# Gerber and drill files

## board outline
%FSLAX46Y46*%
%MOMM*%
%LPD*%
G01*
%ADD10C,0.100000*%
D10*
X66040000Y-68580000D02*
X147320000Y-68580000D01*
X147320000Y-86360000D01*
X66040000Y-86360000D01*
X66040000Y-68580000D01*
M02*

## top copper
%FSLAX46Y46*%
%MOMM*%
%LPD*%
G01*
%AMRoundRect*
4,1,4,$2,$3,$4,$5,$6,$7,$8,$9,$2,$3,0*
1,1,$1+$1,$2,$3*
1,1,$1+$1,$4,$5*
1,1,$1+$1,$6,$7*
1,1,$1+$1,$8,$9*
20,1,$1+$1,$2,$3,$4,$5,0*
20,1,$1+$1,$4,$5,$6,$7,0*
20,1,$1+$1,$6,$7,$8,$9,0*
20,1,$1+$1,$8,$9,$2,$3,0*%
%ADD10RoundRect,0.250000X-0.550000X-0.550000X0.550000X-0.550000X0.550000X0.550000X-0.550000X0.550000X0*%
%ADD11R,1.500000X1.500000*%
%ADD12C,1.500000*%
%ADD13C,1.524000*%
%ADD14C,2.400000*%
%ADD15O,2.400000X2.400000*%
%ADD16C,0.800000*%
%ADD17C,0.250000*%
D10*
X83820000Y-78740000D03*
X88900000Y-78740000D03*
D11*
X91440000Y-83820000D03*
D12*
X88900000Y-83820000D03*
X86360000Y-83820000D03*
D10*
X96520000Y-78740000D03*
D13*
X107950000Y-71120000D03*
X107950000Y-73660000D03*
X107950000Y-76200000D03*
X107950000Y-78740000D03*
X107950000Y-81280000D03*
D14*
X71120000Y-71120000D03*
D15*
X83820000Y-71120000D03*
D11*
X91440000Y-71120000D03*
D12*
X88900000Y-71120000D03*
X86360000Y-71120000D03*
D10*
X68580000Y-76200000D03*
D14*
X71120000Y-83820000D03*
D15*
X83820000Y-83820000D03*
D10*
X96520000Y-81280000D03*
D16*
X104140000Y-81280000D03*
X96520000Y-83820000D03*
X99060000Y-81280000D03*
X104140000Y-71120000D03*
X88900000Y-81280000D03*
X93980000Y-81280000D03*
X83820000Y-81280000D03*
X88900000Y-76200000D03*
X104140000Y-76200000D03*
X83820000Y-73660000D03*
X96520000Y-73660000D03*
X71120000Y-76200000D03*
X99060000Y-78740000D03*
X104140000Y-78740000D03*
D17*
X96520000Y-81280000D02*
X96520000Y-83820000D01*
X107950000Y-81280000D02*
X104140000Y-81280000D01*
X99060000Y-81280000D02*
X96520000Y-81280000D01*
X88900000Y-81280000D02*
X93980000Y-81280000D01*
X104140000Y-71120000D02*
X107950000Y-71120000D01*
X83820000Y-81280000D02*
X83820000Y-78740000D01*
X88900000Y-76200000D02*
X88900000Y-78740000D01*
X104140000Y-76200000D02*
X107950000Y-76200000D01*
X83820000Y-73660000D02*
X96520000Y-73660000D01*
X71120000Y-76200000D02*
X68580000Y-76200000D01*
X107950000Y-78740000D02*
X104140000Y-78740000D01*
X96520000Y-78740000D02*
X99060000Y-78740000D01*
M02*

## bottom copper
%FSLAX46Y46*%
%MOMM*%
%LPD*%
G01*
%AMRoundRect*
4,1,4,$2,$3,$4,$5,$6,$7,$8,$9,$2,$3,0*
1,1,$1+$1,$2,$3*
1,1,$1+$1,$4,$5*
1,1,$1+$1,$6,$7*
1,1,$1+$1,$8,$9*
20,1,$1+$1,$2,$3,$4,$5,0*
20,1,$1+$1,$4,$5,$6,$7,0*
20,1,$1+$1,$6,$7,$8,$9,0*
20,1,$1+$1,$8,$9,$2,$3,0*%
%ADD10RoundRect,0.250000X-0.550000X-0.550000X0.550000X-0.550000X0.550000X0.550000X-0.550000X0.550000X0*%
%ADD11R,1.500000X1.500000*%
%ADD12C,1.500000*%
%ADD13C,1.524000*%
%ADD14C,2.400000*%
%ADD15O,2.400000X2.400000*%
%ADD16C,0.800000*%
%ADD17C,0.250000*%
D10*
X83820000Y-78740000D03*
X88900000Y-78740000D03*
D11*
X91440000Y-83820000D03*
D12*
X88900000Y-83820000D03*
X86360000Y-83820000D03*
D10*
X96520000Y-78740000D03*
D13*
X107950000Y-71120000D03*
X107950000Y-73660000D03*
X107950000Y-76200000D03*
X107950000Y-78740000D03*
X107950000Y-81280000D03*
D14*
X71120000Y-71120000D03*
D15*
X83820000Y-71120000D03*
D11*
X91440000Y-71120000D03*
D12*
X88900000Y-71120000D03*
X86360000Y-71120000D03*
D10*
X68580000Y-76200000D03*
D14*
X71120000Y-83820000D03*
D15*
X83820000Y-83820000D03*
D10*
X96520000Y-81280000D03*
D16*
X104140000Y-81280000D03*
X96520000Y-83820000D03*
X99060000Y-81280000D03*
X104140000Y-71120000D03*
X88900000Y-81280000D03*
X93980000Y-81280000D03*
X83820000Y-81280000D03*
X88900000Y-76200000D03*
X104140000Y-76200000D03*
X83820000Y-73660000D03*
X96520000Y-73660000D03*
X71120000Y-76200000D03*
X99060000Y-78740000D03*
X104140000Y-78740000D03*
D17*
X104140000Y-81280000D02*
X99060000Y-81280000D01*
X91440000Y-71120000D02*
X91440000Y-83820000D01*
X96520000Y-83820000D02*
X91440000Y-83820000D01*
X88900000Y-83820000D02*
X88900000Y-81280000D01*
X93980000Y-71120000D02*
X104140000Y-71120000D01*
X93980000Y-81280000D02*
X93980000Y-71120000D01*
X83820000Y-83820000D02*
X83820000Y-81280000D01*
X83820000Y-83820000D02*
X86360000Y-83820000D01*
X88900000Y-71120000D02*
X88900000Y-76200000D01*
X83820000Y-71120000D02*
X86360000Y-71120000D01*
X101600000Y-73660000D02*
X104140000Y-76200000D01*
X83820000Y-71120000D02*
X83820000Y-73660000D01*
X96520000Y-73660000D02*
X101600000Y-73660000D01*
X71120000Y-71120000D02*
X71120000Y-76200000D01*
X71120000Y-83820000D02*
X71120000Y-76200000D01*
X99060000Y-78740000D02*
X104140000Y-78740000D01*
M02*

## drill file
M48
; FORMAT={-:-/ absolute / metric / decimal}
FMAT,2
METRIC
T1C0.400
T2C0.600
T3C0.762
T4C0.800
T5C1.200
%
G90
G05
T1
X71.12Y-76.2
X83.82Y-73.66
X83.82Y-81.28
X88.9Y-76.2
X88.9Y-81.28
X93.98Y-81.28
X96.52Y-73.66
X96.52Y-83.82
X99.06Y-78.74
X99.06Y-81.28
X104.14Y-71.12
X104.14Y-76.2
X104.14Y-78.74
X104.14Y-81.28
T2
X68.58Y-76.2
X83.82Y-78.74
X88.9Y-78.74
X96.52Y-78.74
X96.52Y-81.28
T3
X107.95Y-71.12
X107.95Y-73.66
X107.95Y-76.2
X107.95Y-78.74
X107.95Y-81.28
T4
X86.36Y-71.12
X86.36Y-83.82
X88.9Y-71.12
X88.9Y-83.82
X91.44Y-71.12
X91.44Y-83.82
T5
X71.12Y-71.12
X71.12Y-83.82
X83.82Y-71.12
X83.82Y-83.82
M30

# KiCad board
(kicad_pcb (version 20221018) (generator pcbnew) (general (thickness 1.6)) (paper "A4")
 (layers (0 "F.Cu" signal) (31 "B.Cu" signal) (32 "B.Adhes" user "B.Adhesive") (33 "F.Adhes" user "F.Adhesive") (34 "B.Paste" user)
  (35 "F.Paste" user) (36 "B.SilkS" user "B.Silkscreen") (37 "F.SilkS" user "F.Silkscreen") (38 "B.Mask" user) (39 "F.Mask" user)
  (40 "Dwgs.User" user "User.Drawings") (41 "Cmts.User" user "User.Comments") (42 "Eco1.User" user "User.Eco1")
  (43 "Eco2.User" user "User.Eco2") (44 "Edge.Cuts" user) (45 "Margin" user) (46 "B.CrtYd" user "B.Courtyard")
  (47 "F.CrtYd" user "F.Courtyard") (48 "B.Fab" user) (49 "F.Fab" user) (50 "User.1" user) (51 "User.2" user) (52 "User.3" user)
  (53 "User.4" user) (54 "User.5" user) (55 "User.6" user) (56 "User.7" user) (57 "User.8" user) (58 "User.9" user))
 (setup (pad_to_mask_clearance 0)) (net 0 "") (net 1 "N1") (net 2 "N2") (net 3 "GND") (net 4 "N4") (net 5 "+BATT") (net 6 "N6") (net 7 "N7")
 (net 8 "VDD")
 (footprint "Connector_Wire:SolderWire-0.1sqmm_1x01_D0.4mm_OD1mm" (layer "F.Cu") (at 83.82 78.74)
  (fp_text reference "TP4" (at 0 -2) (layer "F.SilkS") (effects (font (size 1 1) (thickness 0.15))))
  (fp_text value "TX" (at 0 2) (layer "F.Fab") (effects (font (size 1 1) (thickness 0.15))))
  (pad "1" thru_hole roundrect (at 0 0) (size 1.6 1.6) (drill 0.6) (layers "*.Cu" "*.Mask") (roundrect_rratio 0.15625) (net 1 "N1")))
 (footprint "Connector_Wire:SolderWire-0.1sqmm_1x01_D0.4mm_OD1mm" (layer "F.Cu") (at 88.9 78.74)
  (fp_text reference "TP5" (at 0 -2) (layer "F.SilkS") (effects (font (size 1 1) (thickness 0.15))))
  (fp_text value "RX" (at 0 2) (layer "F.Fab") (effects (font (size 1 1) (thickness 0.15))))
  (pad "1" thru_hole roundrect (at 0 0) (size 1.6 1.6) (drill 0.6) (layers "*.Cu" "*.Mask") (roundrect_rratio 0.15625) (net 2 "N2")))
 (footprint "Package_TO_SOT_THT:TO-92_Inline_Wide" (layer "F.Cu") (at 91.44 83.82 180)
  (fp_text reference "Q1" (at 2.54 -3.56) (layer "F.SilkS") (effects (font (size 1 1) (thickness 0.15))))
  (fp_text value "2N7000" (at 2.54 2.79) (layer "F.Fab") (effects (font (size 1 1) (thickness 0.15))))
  (pad "1" thru_hole rect (at 0 0 180) (size 1.5 1.5) (drill 0.8) (layers "*.Cu" "*.Mask") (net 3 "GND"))
  (pad "2" thru_hole circle (at 2.54 0 180) (size 1.5 1.5) (drill 0.8) (layers "*.Cu" "*.Mask") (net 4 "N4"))
  (pad "3" thru_hole circle (at 5.08 0 180) (size 1.5 1.5) (drill 0.8) (layers "*.Cu" "*.Mask") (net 1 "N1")))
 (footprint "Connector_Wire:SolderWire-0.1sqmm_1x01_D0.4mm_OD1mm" (layer "F.Cu") (at 96.52 78.74)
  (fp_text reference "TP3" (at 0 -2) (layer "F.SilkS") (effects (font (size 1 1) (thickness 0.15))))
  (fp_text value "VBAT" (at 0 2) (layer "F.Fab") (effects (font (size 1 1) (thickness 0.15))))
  (pad "1" thru_hole roundrect (at 0 0) (size 1.6 1.6) (drill 0.6) (layers "*.Cu" "*.Mask") (roundrect_rratio 0.15625) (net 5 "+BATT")))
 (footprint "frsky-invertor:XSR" (layer "F.Cu") (at 107.95 71.12)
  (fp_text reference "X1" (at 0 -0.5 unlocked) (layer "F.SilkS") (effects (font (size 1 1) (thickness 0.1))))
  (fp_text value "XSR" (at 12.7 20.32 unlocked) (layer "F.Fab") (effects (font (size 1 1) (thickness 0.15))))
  (pad "1" thru_hole circle (at 0 0) (size 1.524 1.524) (drill 0.762) (layers "*.Cu" "*.Mask") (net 4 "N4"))
  (pad "2" thru_hole circle (at 0 2.54) (size 1.524 1.524) (drill 0.762) (layers "*.Cu" "*.Mask") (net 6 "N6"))
  (pad "3" thru_hole circle (at 0 5.08) (size 1.524 1.524) (drill 0.762) (layers "*.Cu" "*.Mask") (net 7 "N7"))
  (pad "4" thru_hole circle (at 0 7.62) (size 1.524 1.524) (drill 0.762) (layers "*.Cu" "*.Mask") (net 5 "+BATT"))
  (pad "5" thru_hole circle (at 0 10.16) (size 1.524 1.524) (drill 0.762) (layers "*.Cu" "*.Mask") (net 3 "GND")))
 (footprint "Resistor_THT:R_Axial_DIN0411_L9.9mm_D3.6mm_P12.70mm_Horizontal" (layer "F.Cu") (at 71.12 71.12)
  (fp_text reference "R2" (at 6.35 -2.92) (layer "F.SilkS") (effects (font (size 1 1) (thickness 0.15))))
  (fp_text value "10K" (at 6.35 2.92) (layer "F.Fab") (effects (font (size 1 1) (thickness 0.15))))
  (pad "1" thru_hole circle (at 0 0) (size 2.4 2.4) (drill 1.2) (layers "*.Cu" "*.Mask") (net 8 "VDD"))
  (pad "2" thru_hole oval (at 12.7 0) (size 2.4 2.4) (drill 1.2) (layers "*.Cu" "*.Mask") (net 7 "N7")))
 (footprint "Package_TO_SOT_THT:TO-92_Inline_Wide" (layer "F.Cu") (at 91.44 71.12 180)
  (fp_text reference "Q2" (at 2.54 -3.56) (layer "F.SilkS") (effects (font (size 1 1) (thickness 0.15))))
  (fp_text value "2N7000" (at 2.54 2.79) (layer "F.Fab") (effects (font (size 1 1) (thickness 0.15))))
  (pad "1" thru_hole rect (at 0 0 180) (size 1.5 1.5) (drill 0.8) (layers "*.Cu" "*.Mask") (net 3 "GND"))
  (pad "2" thru_hole circle (at 2.54 0 180) (size 1.5 1.5) (drill 0.8) (layers "*.Cu" "*.Mask") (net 2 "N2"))
  (pad "3" thru_hole circle (at 5.08 0 180) (size 1.5 1.5) (drill 0.8) (layers "*.Cu" "*.Mask") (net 7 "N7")))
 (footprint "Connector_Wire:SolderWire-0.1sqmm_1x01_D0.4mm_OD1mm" (layer "F.Cu") (at 68.58 76.2)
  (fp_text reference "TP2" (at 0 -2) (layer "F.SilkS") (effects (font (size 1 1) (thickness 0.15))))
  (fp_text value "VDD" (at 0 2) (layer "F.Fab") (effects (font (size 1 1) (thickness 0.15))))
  (pad "1" thru_hole roundrect (at 0 0) (size 1.6 1.6) (drill 0.6) (layers "*.Cu" "*.Mask") (roundrect_rratio 0.15625) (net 8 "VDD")))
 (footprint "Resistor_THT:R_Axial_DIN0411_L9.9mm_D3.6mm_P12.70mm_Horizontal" (layer "F.Cu") (at 71.12 83.82)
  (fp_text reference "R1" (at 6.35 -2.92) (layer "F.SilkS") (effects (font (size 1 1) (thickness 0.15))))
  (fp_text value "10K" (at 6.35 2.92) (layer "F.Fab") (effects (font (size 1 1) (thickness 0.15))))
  (pad "1" thru_hole circle (at 0 0) (size 2.4 2.4) (drill 1.2) (layers "*.Cu" "*.Mask") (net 8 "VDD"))
  (pad "2" thru_hole oval (at 12.7 0) (size 2.4 2.4) (drill 1.2) (layers "*.Cu" "*.Mask") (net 1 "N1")))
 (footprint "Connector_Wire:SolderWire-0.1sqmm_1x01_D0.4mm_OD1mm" (layer "F.Cu") (at 96.52 81.28)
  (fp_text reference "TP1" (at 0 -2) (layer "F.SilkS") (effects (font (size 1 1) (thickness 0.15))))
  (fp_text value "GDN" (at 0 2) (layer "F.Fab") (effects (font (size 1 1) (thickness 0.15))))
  (pad "1" thru_hole roundrect (at 0 0) (size 1.6 1.6) (drill 0.6) (layers "*.Cu" "*.Mask") (roundrect_rratio 0.15625) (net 3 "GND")))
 (gr_rect (start 66.04 68.58) (end 147.32 86.36) (stroke (width 0.1) (type default)) (fill none) (layer "Edge.Cuts"))
 (segment (start 96.52 81.28) (end 96.52 83.82) (width 0.25) (layer "F.Cu") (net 3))
 (segment (start 107.95 81.28) (end 104.14 81.28) (width 0.25) (layer "F.Cu") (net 3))
 (segment (start 99.06 81.28) (end 96.52 81.28) (width 0.25) (layer "F.Cu") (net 3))
 (via (at 104.14 81.28) (size 0.8) (drill 0.4) (layers "F.Cu" "B.Cu") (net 3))
 (via (at 96.52 83.82) (size 0.8) (drill 0.4) (layers "F.Cu" "B.Cu") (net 3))
 (via (at 99.06 81.28) (size 0.8) (drill 0.4) (layers "F.Cu" "B.Cu") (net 3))
 (segment (start 104.14 81.28) (end 99.06 81.28) (width 0.25) (layer "B.Cu") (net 3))
 (segment (start 91.44 71.12) (end 91.44 83.82) (width 0.25) (layer "B.Cu") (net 3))
 (segment (start 96.52 83.82) (end 91.44 83.82) (width 0.25) (layer "B.Cu") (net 3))
 (segment (start 88.9 81.28) (end 93.98 81.28) (width 0.25) (layer "F.Cu") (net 4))
 (segment (start 104.14 71.12) (end 107.95 71.12) (width 0.25) (layer "F.Cu") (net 4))
 (via (at 104.14 71.12) (size 0.8) (drill 0.4) (layers "F.Cu" "B.Cu") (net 4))
 (via (at 88.9 81.28) (size 0.8) (drill 0.4) (layers "F.Cu" "B.Cu") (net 4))
 (via (at 93.98 81.28) (size 0.8) (drill 0.4) (layers "F.Cu" "B.Cu") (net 4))
 (segment (start 88.9 83.82) (end 88.9 81.28) (width 0.25) (layer "B.Cu") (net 4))
 (segment (start 93.98 71.12) (end 104.14 71.12) (width 0.25) (layer "B.Cu") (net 4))
 (segment (start 93.98 81.28) (end 93.98 71.12) (width 0.25) (layer "B.Cu") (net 4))
 (segment (start 83.82 81.28) (end 83.82 78.74) (width 0.25) (layer "F.Cu") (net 1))
 (via (at 83.82 81.28) (size 0.8) (drill 0.4) (layers "F.Cu" "B.Cu") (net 1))
 (segment (start 83.82 83.82) (end 83.82 81.28) (width 0.25) (layer "B.Cu") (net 1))
 (segment (start 83.82 83.82) (end 86.36 83.82) (width 0.25) (layer "B.Cu") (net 1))
 (segment (start 88.9 76.2) (end 88.9 78.74) (width 0.25) (layer "F.Cu") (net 2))
 (via (at 88.9 76.2) (size 0.8) (drill 0.4) (layers "F.Cu" "B.Cu") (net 2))
 (segment (start 88.9 71.12) (end 88.9 76.2) (width 0.25) (layer "B.Cu") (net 2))
 (segment (start 104.14 76.2) (end 107.95 76.2) (width 0.25) (layer "F.Cu") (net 7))
 (segment (start 83.82 73.66) (end 96.52 73.66) (width 0.25) (layer "F.Cu") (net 7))
 (via (at 104.14 76.2) (size 0.8) (drill 0.4) (layers "F.Cu" "B.Cu") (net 7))
 (via (at 83.82 73.66) (size 0.8) (drill 0.4) (layers "F.Cu" "B.Cu") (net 7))
 (via (at 96.52 73.66) (size 0.8) (drill 0.4) (layers "F.Cu" "B.Cu") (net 7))
 (segment (start 83.82 71.12) (end 86.36 71.12) (width 0.25) (layer "B.Cu") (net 7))
 (segment (start 101.6 73.66) (end 104.14 76.2) (width 0.25) (layer "B.Cu") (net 7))
 (segment (start 83.82 71.12) (end 83.82 73.66) (width 0.25) (layer "B.Cu") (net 7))
 (segment (start 96.52 73.66) (end 101.6 73.66) (width 0.25) (layer "B.Cu") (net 7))
 (segment (start 71.12 76.2) (end 68.58 76.2) (width 0.25) (layer "F.Cu") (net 8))
 (via (at 71.12 76.2) (size 0.8) (drill 0.4) (layers "F.Cu" "B.Cu") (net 8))
 (segment (start 71.12 71.12) (end 71.12 76.2) (width 0.25) (layer "B.Cu") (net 8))
 (segment (start 71.12 83.82) (end 71.12 76.2) (width 0.25) (layer "B.Cu") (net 8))
 (segment (start 107.95 78.74) (end 104.14 78.74) (width 0.25) (layer "F.Cu") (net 5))
 (segment (start 96.52 78.74) (end 99.06 78.74) (width 0.25) (layer "F.Cu") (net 5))
 (via (at 99.06 78.74) (size 0.8) (drill 0.4) (layers "F.Cu" "B.Cu") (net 5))
 (via (at 104.14 78.74) (size 0.8) (drill 0.4) (layers "F.Cu" "B.Cu") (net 5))
 (segment (start 99.06 78.74) (end 104.14 78.74) (width 0.25) (layer "B.Cu") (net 5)))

